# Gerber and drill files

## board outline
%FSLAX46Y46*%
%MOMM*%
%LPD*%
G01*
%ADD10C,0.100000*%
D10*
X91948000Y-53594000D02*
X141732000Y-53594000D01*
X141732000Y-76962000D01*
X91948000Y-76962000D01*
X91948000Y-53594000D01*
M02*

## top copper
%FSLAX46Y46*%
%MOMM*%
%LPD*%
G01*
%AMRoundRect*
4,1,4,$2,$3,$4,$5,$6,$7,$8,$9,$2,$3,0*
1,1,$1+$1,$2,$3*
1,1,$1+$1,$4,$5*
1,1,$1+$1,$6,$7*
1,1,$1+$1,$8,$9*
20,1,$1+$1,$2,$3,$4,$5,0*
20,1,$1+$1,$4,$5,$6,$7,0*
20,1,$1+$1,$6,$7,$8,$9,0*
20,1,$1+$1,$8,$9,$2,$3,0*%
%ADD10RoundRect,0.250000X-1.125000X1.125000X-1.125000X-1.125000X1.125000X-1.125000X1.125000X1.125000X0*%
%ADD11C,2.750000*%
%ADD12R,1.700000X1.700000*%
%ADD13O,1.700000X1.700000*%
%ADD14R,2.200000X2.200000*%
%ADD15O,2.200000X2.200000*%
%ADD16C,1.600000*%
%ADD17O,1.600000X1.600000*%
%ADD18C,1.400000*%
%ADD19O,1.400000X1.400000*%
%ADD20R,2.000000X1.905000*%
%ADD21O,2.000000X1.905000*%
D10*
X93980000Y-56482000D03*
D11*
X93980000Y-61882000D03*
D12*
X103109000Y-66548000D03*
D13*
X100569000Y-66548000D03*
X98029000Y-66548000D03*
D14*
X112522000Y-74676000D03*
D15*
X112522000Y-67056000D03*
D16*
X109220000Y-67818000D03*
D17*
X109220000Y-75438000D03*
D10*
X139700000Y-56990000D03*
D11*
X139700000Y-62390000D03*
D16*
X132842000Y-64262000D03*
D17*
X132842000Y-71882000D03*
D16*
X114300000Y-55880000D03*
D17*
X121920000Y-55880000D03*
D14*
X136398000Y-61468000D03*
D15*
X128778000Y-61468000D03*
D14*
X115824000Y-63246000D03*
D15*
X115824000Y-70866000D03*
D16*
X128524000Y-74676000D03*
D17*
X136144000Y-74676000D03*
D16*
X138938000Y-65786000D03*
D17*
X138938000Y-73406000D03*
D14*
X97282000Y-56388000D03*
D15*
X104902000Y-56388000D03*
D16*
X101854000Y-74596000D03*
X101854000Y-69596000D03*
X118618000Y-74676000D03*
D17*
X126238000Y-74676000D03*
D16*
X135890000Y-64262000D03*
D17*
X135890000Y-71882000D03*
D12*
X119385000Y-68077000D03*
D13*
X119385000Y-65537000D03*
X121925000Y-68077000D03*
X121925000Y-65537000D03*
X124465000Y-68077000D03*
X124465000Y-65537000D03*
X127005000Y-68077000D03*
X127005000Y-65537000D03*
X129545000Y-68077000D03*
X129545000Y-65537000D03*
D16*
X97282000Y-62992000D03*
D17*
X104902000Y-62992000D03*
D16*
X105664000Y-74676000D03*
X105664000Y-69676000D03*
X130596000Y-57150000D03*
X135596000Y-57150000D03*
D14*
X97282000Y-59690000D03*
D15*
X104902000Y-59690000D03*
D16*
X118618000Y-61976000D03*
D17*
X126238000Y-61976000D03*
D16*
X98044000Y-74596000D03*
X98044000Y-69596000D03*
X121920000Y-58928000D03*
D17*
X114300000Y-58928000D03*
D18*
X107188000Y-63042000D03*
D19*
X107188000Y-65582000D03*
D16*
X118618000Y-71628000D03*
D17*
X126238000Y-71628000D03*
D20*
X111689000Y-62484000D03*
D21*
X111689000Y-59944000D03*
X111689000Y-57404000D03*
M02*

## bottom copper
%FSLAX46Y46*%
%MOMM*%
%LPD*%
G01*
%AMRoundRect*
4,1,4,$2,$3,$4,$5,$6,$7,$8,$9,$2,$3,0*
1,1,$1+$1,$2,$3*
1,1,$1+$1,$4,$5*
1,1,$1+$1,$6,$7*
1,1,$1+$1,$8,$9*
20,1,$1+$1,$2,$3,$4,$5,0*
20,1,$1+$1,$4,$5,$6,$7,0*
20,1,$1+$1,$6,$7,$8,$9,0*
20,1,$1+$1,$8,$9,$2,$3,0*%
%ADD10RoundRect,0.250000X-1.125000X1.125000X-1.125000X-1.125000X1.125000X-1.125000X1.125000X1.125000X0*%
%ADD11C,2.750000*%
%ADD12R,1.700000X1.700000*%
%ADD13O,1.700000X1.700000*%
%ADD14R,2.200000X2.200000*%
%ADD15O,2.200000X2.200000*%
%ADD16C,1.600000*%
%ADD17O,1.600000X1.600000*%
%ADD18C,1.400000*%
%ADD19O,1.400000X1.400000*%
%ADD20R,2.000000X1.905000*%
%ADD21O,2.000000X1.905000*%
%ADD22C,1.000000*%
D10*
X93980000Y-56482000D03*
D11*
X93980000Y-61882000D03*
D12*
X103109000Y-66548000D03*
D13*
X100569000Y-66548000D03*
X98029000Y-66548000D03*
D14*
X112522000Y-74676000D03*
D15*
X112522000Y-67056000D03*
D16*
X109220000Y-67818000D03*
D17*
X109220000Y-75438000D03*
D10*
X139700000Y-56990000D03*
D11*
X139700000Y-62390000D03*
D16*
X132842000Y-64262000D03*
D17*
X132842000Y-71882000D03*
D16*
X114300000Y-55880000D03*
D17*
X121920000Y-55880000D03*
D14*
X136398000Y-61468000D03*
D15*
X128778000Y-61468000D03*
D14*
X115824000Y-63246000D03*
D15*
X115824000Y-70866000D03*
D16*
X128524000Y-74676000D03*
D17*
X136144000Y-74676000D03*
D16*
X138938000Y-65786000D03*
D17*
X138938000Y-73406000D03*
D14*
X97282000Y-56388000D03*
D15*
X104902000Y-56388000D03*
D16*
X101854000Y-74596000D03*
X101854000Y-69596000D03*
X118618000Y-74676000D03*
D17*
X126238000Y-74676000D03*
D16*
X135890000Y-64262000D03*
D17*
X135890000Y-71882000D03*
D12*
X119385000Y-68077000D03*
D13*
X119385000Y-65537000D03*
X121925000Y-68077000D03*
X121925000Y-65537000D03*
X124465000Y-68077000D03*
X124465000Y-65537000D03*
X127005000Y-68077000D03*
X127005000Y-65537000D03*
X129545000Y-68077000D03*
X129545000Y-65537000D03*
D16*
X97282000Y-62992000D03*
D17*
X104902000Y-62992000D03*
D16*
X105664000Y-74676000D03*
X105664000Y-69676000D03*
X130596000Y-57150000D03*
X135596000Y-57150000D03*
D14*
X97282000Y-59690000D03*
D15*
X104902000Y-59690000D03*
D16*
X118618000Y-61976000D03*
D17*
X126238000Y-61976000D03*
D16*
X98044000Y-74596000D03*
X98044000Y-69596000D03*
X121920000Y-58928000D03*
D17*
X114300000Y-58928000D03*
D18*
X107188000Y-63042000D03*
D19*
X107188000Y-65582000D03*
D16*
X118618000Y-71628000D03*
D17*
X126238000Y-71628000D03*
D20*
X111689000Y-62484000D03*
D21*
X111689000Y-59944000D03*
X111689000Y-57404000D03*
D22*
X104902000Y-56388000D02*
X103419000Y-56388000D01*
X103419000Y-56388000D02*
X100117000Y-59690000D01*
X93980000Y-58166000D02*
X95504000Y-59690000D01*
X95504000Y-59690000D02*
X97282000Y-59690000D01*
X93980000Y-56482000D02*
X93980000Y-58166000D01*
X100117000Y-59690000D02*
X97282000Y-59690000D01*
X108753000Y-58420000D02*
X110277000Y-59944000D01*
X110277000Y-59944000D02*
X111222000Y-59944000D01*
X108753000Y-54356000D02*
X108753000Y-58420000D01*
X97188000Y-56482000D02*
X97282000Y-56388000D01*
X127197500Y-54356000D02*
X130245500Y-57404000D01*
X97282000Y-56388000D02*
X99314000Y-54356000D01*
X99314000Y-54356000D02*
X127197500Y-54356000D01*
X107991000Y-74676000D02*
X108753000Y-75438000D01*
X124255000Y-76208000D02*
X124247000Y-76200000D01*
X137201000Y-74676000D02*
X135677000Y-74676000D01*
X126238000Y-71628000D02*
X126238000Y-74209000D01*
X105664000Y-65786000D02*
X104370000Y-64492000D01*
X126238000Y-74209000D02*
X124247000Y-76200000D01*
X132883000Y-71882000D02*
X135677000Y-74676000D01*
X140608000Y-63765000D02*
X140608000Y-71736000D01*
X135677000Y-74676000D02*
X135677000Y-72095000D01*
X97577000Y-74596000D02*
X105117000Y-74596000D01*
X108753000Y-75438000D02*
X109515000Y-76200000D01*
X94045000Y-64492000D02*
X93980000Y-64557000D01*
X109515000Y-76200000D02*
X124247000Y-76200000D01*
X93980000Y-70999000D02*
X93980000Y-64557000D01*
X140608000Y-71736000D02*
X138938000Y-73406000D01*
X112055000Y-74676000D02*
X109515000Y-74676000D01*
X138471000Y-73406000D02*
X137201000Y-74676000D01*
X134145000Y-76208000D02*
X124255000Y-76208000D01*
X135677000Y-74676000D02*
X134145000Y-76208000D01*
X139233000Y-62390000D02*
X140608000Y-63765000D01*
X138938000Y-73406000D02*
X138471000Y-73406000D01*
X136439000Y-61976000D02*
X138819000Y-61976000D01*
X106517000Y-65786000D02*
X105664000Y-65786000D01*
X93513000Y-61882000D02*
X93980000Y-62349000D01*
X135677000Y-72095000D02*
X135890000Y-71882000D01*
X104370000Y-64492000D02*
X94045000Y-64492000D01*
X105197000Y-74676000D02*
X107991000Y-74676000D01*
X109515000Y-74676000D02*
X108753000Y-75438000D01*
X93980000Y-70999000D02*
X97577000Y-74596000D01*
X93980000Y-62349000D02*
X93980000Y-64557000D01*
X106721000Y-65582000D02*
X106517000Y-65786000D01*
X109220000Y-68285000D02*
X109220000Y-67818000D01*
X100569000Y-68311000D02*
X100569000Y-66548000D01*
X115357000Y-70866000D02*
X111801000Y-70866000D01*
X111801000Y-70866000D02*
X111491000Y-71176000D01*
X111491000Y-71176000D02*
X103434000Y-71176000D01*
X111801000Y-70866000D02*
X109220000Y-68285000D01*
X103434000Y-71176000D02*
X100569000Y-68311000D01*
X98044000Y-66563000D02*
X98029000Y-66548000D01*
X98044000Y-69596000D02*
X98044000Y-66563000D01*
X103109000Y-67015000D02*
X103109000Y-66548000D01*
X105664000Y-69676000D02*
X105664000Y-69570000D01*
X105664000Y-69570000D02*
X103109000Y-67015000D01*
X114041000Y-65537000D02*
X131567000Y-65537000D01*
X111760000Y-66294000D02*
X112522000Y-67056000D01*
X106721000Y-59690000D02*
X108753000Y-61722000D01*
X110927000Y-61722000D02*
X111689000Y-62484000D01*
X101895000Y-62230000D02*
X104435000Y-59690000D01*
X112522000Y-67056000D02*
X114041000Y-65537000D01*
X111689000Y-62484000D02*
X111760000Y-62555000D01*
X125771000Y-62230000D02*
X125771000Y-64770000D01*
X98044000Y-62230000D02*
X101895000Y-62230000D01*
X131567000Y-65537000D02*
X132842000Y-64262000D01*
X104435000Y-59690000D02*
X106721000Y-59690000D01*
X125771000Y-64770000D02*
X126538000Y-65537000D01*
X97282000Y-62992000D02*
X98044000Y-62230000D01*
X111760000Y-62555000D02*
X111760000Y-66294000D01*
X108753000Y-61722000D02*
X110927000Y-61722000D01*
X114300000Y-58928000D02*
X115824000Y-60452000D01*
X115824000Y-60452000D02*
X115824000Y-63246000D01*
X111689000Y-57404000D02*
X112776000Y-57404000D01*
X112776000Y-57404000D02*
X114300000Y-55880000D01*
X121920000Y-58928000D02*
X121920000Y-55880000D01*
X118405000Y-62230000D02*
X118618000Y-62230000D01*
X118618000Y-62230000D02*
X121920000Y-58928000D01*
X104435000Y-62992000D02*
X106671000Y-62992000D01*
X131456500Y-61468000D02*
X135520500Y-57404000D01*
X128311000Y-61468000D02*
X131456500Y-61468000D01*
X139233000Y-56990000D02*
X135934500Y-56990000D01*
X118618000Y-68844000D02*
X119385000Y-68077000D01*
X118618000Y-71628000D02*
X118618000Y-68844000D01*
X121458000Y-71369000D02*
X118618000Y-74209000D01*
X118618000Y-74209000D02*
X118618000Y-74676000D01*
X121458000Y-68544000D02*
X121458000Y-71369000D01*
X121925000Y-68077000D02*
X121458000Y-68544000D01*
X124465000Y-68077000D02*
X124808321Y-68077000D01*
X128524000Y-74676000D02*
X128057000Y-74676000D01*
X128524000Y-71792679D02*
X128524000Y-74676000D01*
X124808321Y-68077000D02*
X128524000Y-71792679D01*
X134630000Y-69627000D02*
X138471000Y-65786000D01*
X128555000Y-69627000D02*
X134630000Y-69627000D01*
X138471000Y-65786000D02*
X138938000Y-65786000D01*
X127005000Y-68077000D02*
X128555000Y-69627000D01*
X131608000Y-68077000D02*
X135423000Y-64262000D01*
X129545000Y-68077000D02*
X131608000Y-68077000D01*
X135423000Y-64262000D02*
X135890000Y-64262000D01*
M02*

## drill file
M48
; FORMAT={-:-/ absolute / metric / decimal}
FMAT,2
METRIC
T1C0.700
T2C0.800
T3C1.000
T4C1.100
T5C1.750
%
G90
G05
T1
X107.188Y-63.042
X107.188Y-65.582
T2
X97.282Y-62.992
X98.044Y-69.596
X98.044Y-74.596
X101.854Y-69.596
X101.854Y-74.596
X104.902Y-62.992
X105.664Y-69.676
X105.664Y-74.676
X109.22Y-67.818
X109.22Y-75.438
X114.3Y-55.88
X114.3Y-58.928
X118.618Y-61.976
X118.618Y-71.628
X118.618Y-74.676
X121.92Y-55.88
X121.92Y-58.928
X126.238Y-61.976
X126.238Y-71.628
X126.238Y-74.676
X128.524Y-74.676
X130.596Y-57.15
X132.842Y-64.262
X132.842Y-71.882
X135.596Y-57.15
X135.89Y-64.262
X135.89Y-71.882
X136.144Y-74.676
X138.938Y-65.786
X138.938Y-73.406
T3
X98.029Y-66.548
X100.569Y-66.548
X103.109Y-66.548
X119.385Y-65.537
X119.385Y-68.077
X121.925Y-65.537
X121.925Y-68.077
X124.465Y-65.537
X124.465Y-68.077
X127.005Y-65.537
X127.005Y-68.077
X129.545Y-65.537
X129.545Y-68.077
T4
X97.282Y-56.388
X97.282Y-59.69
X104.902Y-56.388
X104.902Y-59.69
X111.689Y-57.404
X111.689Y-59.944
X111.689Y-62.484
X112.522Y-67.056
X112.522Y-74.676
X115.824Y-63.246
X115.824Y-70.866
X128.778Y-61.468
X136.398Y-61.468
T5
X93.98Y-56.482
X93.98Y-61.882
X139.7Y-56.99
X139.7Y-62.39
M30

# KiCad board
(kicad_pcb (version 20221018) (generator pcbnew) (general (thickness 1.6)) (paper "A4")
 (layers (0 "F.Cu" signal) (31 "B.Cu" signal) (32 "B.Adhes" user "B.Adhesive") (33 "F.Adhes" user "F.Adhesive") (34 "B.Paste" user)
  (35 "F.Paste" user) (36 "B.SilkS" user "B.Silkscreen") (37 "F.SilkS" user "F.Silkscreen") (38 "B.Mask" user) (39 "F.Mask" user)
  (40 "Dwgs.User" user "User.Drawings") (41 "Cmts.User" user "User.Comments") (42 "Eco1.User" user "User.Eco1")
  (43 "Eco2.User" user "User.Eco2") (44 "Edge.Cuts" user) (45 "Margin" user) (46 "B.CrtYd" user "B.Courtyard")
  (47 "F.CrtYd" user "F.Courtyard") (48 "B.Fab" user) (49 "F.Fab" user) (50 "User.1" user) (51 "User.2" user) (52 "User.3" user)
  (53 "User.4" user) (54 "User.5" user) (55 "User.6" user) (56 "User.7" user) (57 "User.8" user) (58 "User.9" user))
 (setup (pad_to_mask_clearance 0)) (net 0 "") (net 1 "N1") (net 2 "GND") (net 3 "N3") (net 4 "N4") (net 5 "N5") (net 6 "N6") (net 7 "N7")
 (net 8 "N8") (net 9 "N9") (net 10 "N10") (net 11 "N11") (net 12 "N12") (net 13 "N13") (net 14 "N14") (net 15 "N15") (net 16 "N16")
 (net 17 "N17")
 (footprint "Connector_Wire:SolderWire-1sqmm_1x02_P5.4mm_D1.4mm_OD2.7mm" (layer "F.Cu") (at 93.98 56.482 -90)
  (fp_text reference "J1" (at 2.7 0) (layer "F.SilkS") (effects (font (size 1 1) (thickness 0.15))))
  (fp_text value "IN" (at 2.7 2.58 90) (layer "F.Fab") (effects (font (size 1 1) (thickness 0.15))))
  (pad "1" thru_hole roundrect (at 0 0 270) (size 2.75 2.75) (drill 1.75) (layers "*.Cu" "*.Mask") (roundrect_rratio 0.090909) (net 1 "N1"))
  (pad "2" thru_hole circle (at 5.4 0 270) (size 2.75 2.75) (drill 1.75) (layers "*.Cu" "*.Mask") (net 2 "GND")))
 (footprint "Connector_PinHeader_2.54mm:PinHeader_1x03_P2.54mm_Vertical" (layer "F.Cu") (at 103.109 66.548 -90)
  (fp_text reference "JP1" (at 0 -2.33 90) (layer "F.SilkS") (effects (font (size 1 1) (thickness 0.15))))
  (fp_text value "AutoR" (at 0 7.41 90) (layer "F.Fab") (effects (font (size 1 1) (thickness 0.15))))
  (pad "1" thru_hole rect (at 0 0 270) (size 1.7 1.7) (drill 1) (layers "*.Cu" "*.Mask") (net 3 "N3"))
  (pad "2" thru_hole oval (at 0 2.54 270) (size 1.7 1.7) (drill 1) (layers "*.Cu" "*.Mask") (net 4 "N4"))
  (pad "3" thru_hole oval (at 0 5.08 270) (size 1.7 1.7) (drill 1) (layers "*.Cu" "*.Mask") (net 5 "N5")))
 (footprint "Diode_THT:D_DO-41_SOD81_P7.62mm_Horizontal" (layer "F.Cu") (at 112.522 74.676 90)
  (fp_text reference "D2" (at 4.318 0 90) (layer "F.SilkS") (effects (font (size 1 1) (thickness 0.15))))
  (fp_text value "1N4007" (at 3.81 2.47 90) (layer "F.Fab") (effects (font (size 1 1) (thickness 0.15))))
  (pad "1" thru_hole rect (at 0 0 90) (size 2.2 2.2) (drill 1.1) (layers "*.Cu" "*.Mask") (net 2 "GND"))
  (pad "2" thru_hole oval (at 7.62 0 90) (size 2.2 2.2) (drill 1.1) (layers "*.Cu" "*.Mask") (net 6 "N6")))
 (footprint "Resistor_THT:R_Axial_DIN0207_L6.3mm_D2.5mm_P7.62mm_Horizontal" (layer "F.Cu") (at 109.22 67.818 -90)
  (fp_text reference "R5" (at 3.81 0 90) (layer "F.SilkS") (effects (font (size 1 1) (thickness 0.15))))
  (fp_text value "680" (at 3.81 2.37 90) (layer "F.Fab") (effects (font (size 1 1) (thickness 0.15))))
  (pad "1" thru_hole circle (at 0 0 270) (size 1.6 1.6) (drill 0.8) (layers "*.Cu" "*.Mask") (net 4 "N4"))
  (pad "2" thru_hole oval (at 7.62 0 270) (size 1.6 1.6) (drill 0.8) (layers "*.Cu" "*.Mask") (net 2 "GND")))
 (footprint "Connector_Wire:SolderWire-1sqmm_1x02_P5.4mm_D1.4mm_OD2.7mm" (layer "F.Cu") (at 139.7 56.99 -90)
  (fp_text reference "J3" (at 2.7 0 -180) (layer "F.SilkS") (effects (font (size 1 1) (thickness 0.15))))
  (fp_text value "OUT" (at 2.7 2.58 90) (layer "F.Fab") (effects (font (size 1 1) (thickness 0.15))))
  (pad "1" thru_hole roundrect (at 0 0 270) (size 2.75 2.75) (drill 1.75) (layers "*.Cu" "*.Mask") (roundrect_rratio 0.090909) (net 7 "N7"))
  (pad "2" thru_hole circle (at 5.4 0 270) (size 2.75 2.75) (drill 1.75) (layers "*.Cu" "*.Mask") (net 2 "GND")))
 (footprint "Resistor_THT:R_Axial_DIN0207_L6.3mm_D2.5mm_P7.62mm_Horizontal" (layer "F.Cu") (at 132.842 64.262 -90)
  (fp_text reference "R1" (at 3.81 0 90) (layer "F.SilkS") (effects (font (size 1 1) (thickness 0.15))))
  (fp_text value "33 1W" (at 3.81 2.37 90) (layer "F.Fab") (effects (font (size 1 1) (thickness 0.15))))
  (pad "1" thru_hole circle (at 0 0 270) (size 1.6 1.6) (drill 0.8) (layers "*.Cu" "*.Mask") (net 6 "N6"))
  (pad "2" thru_hole oval (at 7.62 0 270) (size 1.6 1.6) (drill 0.8) (layers "*.Cu" "*.Mask") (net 2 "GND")))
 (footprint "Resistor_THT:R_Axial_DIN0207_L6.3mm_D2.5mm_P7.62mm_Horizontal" (layer "F.Cu") (at 114.3 55.88)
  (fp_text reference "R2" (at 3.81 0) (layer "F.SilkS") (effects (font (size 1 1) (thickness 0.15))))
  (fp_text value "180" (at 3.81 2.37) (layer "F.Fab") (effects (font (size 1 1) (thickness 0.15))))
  (pad "1" thru_hole circle (at 0 0) (size 1.6 1.6) (drill 0.8) (layers "*.Cu" "*.Mask") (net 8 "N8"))
  (pad "2" thru_hole oval (at 7.62 0) (size 1.6 1.6) (drill 0.8) (layers "*.Cu" "*.Mask") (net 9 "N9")))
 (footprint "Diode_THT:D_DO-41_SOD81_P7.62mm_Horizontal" (layer "F.Cu") (at 136.398 61.468 180)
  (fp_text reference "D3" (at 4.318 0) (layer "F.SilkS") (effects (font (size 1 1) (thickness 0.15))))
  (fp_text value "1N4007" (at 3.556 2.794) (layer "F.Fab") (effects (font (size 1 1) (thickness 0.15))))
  (pad "1" thru_hole rect (at 0 0 180) (size 2.2 2.2) (drill 1.1) (layers "*.Cu" "*.Mask") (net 2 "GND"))
  (pad "2" thru_hole oval (at 7.62 0 180) (size 2.2 2.2) (drill 1.1) (layers "*.Cu" "*.Mask") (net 7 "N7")))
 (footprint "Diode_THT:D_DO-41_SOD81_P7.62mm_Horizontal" (layer "F.Cu") (at 115.824 63.246 -90)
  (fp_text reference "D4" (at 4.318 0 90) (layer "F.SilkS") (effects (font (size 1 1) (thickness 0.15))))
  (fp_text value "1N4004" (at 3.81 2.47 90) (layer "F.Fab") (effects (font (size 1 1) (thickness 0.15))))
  (pad "1" thru_hole rect (at 0 0 270) (size 2.2 2.2) (drill 1.1) (layers "*.Cu" "*.Mask") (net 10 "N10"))
  (pad "2" thru_hole oval (at 7.62 0 270) (size 2.2 2.2) (drill 1.1) (layers "*.Cu" "*.Mask") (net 4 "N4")))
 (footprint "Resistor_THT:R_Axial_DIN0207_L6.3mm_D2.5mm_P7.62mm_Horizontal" (layer "F.Cu") (at 128.524 74.676)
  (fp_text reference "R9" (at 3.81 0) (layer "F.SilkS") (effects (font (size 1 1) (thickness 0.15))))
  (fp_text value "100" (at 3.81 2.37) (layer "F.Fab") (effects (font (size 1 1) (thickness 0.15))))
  (pad "1" thru_hole circle (at 0 0) (size 1.6 1.6) (drill 0.8) (layers "*.Cu" "*.Mask") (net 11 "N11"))
  (pad "2" thru_hole oval (at 7.62 0) (size 1.6 1.6) (drill 0.8) (layers "*.Cu" "*.Mask") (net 2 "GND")))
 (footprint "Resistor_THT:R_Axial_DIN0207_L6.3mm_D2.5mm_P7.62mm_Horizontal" (layer "F.Cu") (at 138.938 65.786 -90)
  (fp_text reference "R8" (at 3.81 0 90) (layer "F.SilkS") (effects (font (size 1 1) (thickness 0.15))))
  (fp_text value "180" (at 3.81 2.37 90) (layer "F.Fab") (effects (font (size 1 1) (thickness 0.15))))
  (pad "1" thru_hole circle (at 0 0 270) (size 1.6 1.6) (drill 0.8) (layers "*.Cu" "*.Mask") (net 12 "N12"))
  (pad "2" thru_hole oval (at 7.62 0 270) (size 1.6 1.6) (drill 0.8) (layers "*.Cu" "*.Mask") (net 2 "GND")))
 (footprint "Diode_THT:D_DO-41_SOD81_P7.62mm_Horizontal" (layer "F.Cu") (at 97.282 56.388)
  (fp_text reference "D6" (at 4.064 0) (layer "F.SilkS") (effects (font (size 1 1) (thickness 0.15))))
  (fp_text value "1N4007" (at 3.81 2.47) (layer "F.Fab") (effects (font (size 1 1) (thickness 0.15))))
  (pad "1" thru_hole rect (at 0 0) (size 2.2 2.2) (drill 1.1) (layers "*.Cu" "*.Mask") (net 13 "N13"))
  (pad "2" thru_hole oval (at 7.62 0) (size 2.2 2.2) (drill 1.1) (layers "*.Cu" "*.Mask") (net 1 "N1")))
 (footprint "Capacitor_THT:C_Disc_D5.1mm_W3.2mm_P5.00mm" (layer "F.Cu") (at 101.854 74.596 90)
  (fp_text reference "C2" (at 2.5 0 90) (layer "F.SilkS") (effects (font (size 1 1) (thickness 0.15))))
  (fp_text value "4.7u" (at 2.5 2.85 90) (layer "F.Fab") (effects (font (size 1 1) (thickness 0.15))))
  (pad "1" thru_hole circle (at 0 0 90) (size 1.6 1.6) (drill 0.8) (layers "*.Cu" "*.Mask") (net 2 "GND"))
  (pad "2" thru_hole circle (at 5 0 90) (size 1.6 1.6) (drill 0.8) (layers "*.Cu" "*.Mask") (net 4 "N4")))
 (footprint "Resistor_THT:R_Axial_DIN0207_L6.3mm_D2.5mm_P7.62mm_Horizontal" (layer "F.Cu") (at 118.618 74.676)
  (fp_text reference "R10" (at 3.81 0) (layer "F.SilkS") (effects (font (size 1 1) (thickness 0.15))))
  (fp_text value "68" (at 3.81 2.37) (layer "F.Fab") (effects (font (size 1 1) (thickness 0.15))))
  (pad "1" thru_hole circle (at 0 0) (size 1.6 1.6) (drill 0.8) (layers "*.Cu" "*.Mask") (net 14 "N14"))
  (pad "2" thru_hole oval (at 7.62 0) (size 1.6 1.6) (drill 0.8) (layers "*.Cu" "*.Mask") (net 2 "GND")))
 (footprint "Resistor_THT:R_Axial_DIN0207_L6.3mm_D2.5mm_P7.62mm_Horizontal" (layer "F.Cu") (at 135.89 64.262 -90)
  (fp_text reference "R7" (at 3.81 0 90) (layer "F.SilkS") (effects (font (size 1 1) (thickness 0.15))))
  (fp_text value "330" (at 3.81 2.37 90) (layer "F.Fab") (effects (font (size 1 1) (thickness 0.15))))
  (pad "1" thru_hole circle (at 0 0 270) (size 1.6 1.6) (drill 0.8) (layers "*.Cu" "*.Mask") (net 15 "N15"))
  (pad "2" thru_hole oval (at 7.62 0 270) (size 1.6 1.6) (drill 0.8) (layers "*.Cu" "*.Mask") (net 2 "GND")))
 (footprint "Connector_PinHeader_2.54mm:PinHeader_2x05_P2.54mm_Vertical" (layer "F.Cu") (at 119.385 68.077 90)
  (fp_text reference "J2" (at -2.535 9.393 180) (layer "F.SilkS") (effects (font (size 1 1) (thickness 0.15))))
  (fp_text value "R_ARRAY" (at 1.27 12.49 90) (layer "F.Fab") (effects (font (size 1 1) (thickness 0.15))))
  (pad "1" thru_hole rect (at 0 0 90) (size 1.7 1.7) (drill 1) (layers "*.Cu" "*.Mask") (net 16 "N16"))
  (pad "2" thru_hole oval (at 2.54 0 90) (size 1.7 1.7) (drill 1) (layers "*.Cu" "*.Mask") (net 6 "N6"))
  (pad "3" thru_hole oval (at 0 2.54 90) (size 1.7 1.7) (drill 1) (layers "*.Cu" "*.Mask") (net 14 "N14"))
  (pad "4" thru_hole oval (at 2.54 2.54 90) (size 1.7 1.7) (drill 1) (layers "*.Cu" "*.Mask") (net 6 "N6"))
  (pad "5" thru_hole oval (at 0 5.08 90) (size 1.7 1.7) (drill 1) (layers "*.Cu" "*.Mask") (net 11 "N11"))
  (pad "6" thru_hole oval (at 2.54 5.08 90) (size 1.7 1.7) (drill 1) (layers "*.Cu" "*.Mask") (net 6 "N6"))
  (pad "7" thru_hole oval (at 0 7.62 90) (size 1.7 1.7) (drill 1) (layers "*.Cu" "*.Mask") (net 12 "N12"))
  (pad "8" thru_hole oval (at 2.54 7.62 90) (size 1.7 1.7) (drill 1) (layers "*.Cu" "*.Mask") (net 6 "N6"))
  (pad "9" thru_hole oval (at 0 10.16 90) (size 1.7 1.7) (drill 1) (layers "*.Cu" "*.Mask") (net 15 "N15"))
  (pad "10" thru_hole oval (at 2.54 10.16 90) (size 1.7 1.7) (drill 1) (layers "*.Cu" "*.Mask") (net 6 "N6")))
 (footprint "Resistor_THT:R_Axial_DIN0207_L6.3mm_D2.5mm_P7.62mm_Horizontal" (layer "F.Cu") (at 97.282 62.992)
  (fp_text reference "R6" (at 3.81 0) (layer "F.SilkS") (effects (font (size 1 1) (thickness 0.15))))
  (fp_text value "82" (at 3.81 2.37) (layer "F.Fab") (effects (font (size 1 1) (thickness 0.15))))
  (pad "1" thru_hole circle (at 0 0) (size 1.6 1.6) (drill 0.8) (layers "*.Cu" "*.Mask") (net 6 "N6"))
  (pad "2" thru_hole oval (at 7.62 0) (size 1.6 1.6) (drill 0.8) (layers "*.Cu" "*.Mask") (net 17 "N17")))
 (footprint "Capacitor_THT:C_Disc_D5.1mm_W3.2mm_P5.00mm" (layer "F.Cu") (at 105.664 74.676 90)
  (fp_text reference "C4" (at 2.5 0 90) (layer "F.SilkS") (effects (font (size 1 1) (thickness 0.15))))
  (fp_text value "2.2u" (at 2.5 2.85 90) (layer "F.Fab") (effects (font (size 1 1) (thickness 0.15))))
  (pad "1" thru_hole circle (at 0 0 90) (size 1.6 1.6) (drill 0.8) (layers "*.Cu" "*.Mask") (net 2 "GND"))
  (pad "2" thru_hole circle (at 5 0 90) (size 1.6 1.6) (drill 0.8) (layers "*.Cu" "*.Mask") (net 3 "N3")))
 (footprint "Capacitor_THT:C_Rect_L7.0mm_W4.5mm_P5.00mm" (layer "F.Cu") (at 130.596 57.15)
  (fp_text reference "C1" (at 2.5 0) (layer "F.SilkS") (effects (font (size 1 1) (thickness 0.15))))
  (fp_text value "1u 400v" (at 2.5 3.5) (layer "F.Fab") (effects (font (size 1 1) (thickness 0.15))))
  (pad "1" thru_hole circle (at 0 0) (size 1.6 1.6) (drill 0.8) (layers "*.Cu" "*.Mask") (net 13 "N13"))
  (pad "2" thru_hole circle (at 5 0) (size 1.6 1.6) (drill 0.8) (layers "*.Cu" "*.Mask") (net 7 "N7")))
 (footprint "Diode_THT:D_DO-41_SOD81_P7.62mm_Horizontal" (layer "F.Cu") (at 97.282 59.69)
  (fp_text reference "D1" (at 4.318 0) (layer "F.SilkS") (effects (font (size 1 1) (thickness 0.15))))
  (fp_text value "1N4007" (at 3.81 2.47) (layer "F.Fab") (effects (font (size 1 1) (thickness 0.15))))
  (pad "1" thru_hole rect (at 0 0) (size 2.2 2.2) (drill 1.1) (layers "*.Cu" "*.Mask") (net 1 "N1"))
  (pad "2" thru_hole oval (at 7.62 0) (size 2.2 2.2) (drill 1.1) (layers "*.Cu" "*.Mask") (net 6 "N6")))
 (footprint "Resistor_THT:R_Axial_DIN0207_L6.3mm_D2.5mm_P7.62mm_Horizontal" (layer "F.Cu") (at 118.618 61.976)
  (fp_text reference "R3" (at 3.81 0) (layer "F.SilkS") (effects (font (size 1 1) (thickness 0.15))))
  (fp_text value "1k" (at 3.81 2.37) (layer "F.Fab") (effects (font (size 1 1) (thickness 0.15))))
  (pad "1" thru_hole circle (at 0 0) (size 1.6 1.6) (drill 0.8) (layers "*.Cu" "*.Mask") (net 9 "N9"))
  (pad "2" thru_hole oval (at 7.62 0) (size 1.6 1.6) (drill 0.8) (layers "*.Cu" "*.Mask") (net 6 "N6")))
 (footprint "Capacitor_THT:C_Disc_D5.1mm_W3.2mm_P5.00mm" (layer "F.Cu") (at 98.044 74.596 90)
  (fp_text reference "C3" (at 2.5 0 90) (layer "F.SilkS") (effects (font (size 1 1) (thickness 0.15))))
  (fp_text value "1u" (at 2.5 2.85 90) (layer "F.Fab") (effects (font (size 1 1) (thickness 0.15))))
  (pad "1" thru_hole circle (at 0 0 90) (size 1.6 1.6) (drill 0.8) (layers "*.Cu" "*.Mask") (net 2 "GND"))
  (pad "2" thru_hole circle (at 5 0 90) (size 1.6 1.6) (drill 0.8) (layers "*.Cu" "*.Mask") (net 5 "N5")))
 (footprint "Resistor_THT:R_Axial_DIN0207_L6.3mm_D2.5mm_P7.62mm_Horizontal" (layer "F.Cu") (at 121.92 58.928 180)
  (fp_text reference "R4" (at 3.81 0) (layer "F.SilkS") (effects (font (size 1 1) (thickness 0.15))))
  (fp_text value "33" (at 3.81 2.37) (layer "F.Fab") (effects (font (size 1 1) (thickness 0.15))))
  (pad "1" thru_hole circle (at 0 0 180) (size 1.6 1.6) (drill 0.8) (layers "*.Cu" "*.Mask") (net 9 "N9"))
  (pad "2" thru_hole oval (at 7.62 0 180) (size 1.6 1.6) (drill 0.8) (layers "*.Cu" "*.Mask") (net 10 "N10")))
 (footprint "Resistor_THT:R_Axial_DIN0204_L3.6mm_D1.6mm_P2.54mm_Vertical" (layer "F.Cu") (at 107.188 63.042 -90)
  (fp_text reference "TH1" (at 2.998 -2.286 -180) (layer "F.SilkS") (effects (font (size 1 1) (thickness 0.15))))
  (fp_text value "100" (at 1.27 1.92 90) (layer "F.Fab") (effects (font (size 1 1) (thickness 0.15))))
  (pad "1" thru_hole circle (at 0 0 270) (size 1.4 1.4) (drill 0.7) (layers "*.Cu" "*.Mask") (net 17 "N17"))
  (pad "2" thru_hole oval (at 2.54 0 270) (size 1.4 1.4) (drill 0.7) (layers "*.Cu" "*.Mask") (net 2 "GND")))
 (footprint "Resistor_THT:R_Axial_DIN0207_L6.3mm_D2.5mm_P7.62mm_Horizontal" (layer "F.Cu") (at 118.618 71.628)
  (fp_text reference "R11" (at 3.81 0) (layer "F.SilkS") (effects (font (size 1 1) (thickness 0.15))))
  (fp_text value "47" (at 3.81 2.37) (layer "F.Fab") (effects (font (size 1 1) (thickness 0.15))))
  (pad "1" thru_hole circle (at 0 0) (size 1.6 1.6) (drill 0.8) (layers "*.Cu" "*.Mask") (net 16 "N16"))
  (pad "2" thru_hole oval (at 7.62 0) (size 1.6 1.6) (drill 0.8) (layers "*.Cu" "*.Mask") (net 2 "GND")))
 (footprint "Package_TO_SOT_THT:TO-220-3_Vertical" (layer "F.Cu") (at 111.689 62.484 90)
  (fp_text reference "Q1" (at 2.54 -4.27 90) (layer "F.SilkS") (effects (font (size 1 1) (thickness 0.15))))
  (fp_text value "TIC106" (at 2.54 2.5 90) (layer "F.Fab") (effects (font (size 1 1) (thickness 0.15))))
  (pad "1" thru_hole rect (at 0 0 90) (size 1.905 2) (drill 1.1) (layers "*.Cu" "*.Mask") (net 6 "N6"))
  (pad "2" thru_hole oval (at 2.54 0 90) (size 1.905 2) (drill 1.1) (layers "*.Cu" "*.Mask") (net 13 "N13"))
  (pad "3" thru_hole oval (at 5.08 0 90) (size 1.905 2) (drill 1.1) (layers "*.Cu" "*.Mask") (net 8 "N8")))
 (gr_rect (start 91.948 53.594) (end 141.732 76.962) (stroke (width 0.1) (type default)) (fill none) (layer "Edge.Cuts"))
 (segment (start 104.902 56.388) (end 103.419 56.388) (width 1) (layer "B.Cu") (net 1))
 (segment (start 103.419 56.388) (end 100.117 59.69) (width 1) (layer "B.Cu") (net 1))
 (segment (start 93.98 58.166) (end 95.504 59.69) (width 1) (layer "B.Cu") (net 1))
 (segment (start 95.504 59.69) (end 97.282 59.69) (width 1) (layer "B.Cu") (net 1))
 (segment (start 93.98 56.482) (end 93.98 58.166) (width 1) (layer "B.Cu") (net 1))
 (segment (start 100.117 59.69) (end 97.282 59.69) (width 1) (layer "B.Cu") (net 1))
 (segment (start 108.753 58.42) (end 110.277 59.944) (width 1) (layer "B.Cu") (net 13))
 (segment (start 110.277 59.944) (end 111.222 59.944) (width 1) (layer "B.Cu") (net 13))
 (segment (start 108.753 54.356) (end 108.753 58.42) (width 1) (layer "B.Cu") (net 13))
 (segment (start 97.188 56.482) (end 97.282 56.388) (width 1) (layer "B.Cu") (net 13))
 (segment (start 127.1975 54.356) (end 130.2455 57.404) (width 1) (layer "B.Cu") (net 13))
 (segment (start 97.282 56.388) (end 99.314 54.356) (width 1) (layer "B.Cu") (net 13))
 (segment (start 99.314 54.356) (end 127.1975 54.356) (width 1) (layer "B.Cu") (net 13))
 (segment (start 107.991 74.676) (end 108.753 75.438) (width 1) (layer "B.Cu") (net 2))
 (segment (start 124.255 76.208) (end 124.247 76.2) (width 1) (layer "B.Cu") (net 2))
 (segment (start 137.201 74.676) (end 135.677 74.676) (width 1) (layer "B.Cu") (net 2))
 (segment (start 126.238 71.628) (end 126.238 74.209) (width 1) (layer "B.Cu") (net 2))
 (segment (start 105.664 65.786) (end 104.37 64.492) (width 1) (layer "B.Cu") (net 2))
 (segment (start 126.238 74.209) (end 124.247 76.2) (width 1) (layer "B.Cu") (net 2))
 (segment (start 132.883 71.882) (end 135.677 74.676) (width 1) (layer "B.Cu") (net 2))
 (segment (start 140.608 63.765) (end 140.608 71.736) (width 1) (layer "B.Cu") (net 2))
 (segment (start 135.677 74.676) (end 135.677 72.095) (width 1) (layer "B.Cu") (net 2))
 (segment (start 97.577 74.596) (end 105.117 74.596) (width 1) (layer "B.Cu") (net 2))
 (segment (start 108.753 75.438) (end 109.515 76.2) (width 1) (layer "B.Cu") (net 2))
 (segment (start 94.045 64.492) (end 93.98 64.557) (width 1) (layer "B.Cu") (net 2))
 (segment (start 109.515 76.2) (end 124.247 76.2) (width 1) (layer "B.Cu") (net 2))
 (segment (start 93.98 70.999) (end 93.98 64.557) (width 1) (layer "B.Cu") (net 2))
 (segment (start 140.608 71.736) (end 138.938 73.406) (width 1) (layer "B.Cu") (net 2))
 (segment (start 112.055 74.676) (end 109.515 74.676) (width 1) (layer "B.Cu") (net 2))
 (segment (start 138.471 73.406) (end 137.201 74.676) (width 1) (layer "B.Cu") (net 2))
 (segment (start 134.145 76.208) (end 124.255 76.208) (width 1) (layer "B.Cu") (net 2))
 (segment (start 135.677 74.676) (end 134.145 76.208) (width 1) (layer "B.Cu") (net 2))
 (segment (start 139.233 62.39) (end 140.608 63.765) (width 1) (layer "B.Cu") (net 2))
 (segment (start 138.938 73.406) (end 138.471 73.406) (width 1) (layer "B.Cu") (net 2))
 (segment (start 136.439 61.976) (end 138.819 61.976) (width 1) (layer "B.Cu") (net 2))
 (segment (start 106.517 65.786) (end 105.664 65.786) (width 1) (layer "B.Cu") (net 2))
 (segment (start 93.513 61.882) (end 93.98 62.349) (width 1) (layer "B.Cu") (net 2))
 (segment (start 135.677 72.095) (end 135.89 71.882) (width 1) (layer "B.Cu") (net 2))
 (segment (start 104.37 64.492) (end 94.045 64.492) (width 1) (layer "B.Cu") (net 2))
 (segment (start 105.197 74.676) (end 107.991 74.676) (width 1) (layer "B.Cu") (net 2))
 (segment (start 109.515 74.676) (end 108.753 75.438) (width 1) (layer "B.Cu") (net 2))
 (segment (start 93.98 70.999) (end 97.577 74.596) (width 1) (layer "B.Cu") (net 2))
 (segment (start 93.98 62.349) (end 93.98 64.557) (width 1) (layer "B.Cu") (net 2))
 (segment (start 106.721 65.582) (end 106.517 65.786) (width 1) (layer "B.Cu") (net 2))
 (segment (start 109.22 68.285) (end 109.22 67.818) (width 1) (layer "B.Cu") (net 4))
 (segment (start 100.569 68.311) (end 100.569 66.548) (width 1) (layer "B.Cu") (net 4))
 (segment (start 115.357 70.866) (end 111.801 70.866) (width 1) (layer "B.Cu") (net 4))
 (segment (start 111.801 70.866) (end 111.491 71.176) (width 1) (layer "B.Cu") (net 4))
 (segment (start 111.491 71.176) (end 103.434 71.176) (width 1) (layer "B.Cu") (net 4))
 (segment (start 111.801 70.866) (end 109.22 68.285) (width 1) (layer "B.Cu") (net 4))
 (segment (start 103.434 71.176) (end 100.569 68.311) (width 1) (layer "B.Cu") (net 4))
 (segment (start 98.044 66.563) (end 98.029 66.548) (width 1) (layer "B.Cu") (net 5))
 (segment (start 98.044 69.596) (end 98.044 66.563) (width 1) (layer "B.Cu") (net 5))
 (segment (start 103.109 67.015) (end 103.109 66.548) (width 1) (layer "B.Cu") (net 3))
 (segment (start 105.664 69.676) (end 105.664 69.57) (width 1) (layer "B.Cu") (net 3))
 (segment (start 105.664 69.57) (end 103.109 67.015) (width 1) (layer "B.Cu") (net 3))
 (segment (start 114.041 65.537) (end 131.567 65.537) (width 1) (layer "B.Cu") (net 6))
 (segment (start 111.76 66.294) (end 112.522 67.056) (width 1) (layer "B.Cu") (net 6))
 (segment (start 106.721 59.69) (end 108.753 61.722) (width 1) (layer "B.Cu") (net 6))
 (segment (start 110.927 61.722) (end 111.689 62.484) (width 1) (layer "B.Cu") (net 6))
 (segment (start 101.895 62.23) (end 104.435 59.69) (width 1) (layer "B.Cu") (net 6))
 (segment (start 112.522 67.056) (end 114.041 65.537) (width 1) (layer "B.Cu") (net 6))
 (segment (start 111.689 62.484) (end 111.76 62.555) (width 1) (layer "B.Cu") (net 6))
 (segment (start 125.771 62.23) (end 125.771 64.77) (width 1) (layer "B.Cu") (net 6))
 (segment (start 98.044 62.23) (end 101.895 62.23) (width 1) (layer "B.Cu") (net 6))
 (segment (start 131.567 65.537) (end 132.842 64.262) (width 1) (layer "B.Cu") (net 6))
 (segment (start 104.435 59.69) (end 106.721 59.69) (width 1) (layer "B.Cu") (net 6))
 (segment (start 125.771 64.77) (end 126.538 65.537) (width 1) (layer "B.Cu") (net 6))
 (segment (start 97.282 62.992) (end 98.044 62.23) (width 1) (layer "B.Cu") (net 6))
 (segment (start 111.76 62.555) (end 111.76 66.294) (width 1) (layer "B.Cu") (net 6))
 (segment (start 108.753 61.722) (end 110.927 61.722) (width 1) (layer "B.Cu") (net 6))
 (segment (start 114.3 58.928) (end 115.824 60.452) (width 1) (layer "B.Cu") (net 10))
 (segment (start 115.824 60.452) (end 115.824 63.246) (width 1) (layer "B.Cu") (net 10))
 (segment (start 111.689 57.404) (end 112.776 57.404) (width 1) (layer "B.Cu") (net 8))
 (segment (start 112.776 57.404) (end 114.3 55.88) (width 1) (layer "B.Cu") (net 8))
 (segment (start 121.92 58.928) (end 121.92 55.88) (width 1) (layer "B.Cu") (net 9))
 (segment (start 118.405 62.23) (end 118.618 62.23) (width 1) (layer "B.Cu") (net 9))
 (segment (start 118.618 62.23) (end 121.92 58.928) (width 1) (layer "B.Cu") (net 9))
 (segment (start 104.435 62.992) (end 106.671 62.992) (width 1) (layer "B.Cu") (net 17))
 (segment (start 131.4565 61.468) (end 135.5205 57.404) (width 1) (layer "B.Cu") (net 7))
 (segment (start 128.311 61.468) (end 131.4565 61.468) (width 1) (layer "B.Cu") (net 7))
 (segment (start 139.233 56.99) (end 135.9345 56.99) (width 1) (layer "B.Cu") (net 7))
 (segment (start 118.618 68.844) (end 119.385 68.077) (width 1) (layer "B.Cu") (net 16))
 (segment (start 118.618 71.628) (end 118.618 68.844) (width 1) (layer "B.Cu") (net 16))
 (segment (start 121.458 71.369) (end 118.618 74.209) (width 1) (layer "B.Cu") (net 14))
 (segment (start 118.618 74.209) (end 118.618 74.676) (width 1) (layer "B.Cu") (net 14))
 (segment (start 121.458 68.544) (end 121.458 71.369) (width 1) (layer "B.Cu") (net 14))
 (segment (start 121.925 68.077) (end 121.458 68.544) (width 1) (layer "B.Cu") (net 14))
 (segment (start 124.465 68.077) (end 124.808321 68.077) (width 1) (layer "B.Cu") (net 11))
 (segment (start 128.524 74.676) (end 128.057 74.676) (width 1) (layer "B.Cu") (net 11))
 (segment (start 128.524 71.792679) (end 128.524 74.676) (width 1) (layer "B.Cu") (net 11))
 (segment (start 124.808321 68.077) (end 128.524 71.792679) (width 1) (layer "B.Cu") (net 11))
 (segment (start 134.63 69.627) (end 138.471 65.786) (width 1) (layer "B.Cu") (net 12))
 (segment (start 128.555 69.627) (end 134.63 69.627) (width 1) (layer "B.Cu") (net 12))
 (segment (start 138.471 65.786) (end 138.938 65.786) (width 1) (layer "B.Cu") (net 12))
 (segment (start 127.005 68.077) (end 128.555 69.627) (width 1) (layer "B.Cu") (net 12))
 (segment (start 131.608 68.077) (end 135.423 64.262) (width 1) (layer "B.Cu") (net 15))
 (segment (start 129.545 68.077) (end 131.608 68.077) (width 1) (layer "B.Cu") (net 15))
 (segment (start 135.423 64.262) (end 135.89 64.262) (width 1) (layer "B.Cu") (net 15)))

